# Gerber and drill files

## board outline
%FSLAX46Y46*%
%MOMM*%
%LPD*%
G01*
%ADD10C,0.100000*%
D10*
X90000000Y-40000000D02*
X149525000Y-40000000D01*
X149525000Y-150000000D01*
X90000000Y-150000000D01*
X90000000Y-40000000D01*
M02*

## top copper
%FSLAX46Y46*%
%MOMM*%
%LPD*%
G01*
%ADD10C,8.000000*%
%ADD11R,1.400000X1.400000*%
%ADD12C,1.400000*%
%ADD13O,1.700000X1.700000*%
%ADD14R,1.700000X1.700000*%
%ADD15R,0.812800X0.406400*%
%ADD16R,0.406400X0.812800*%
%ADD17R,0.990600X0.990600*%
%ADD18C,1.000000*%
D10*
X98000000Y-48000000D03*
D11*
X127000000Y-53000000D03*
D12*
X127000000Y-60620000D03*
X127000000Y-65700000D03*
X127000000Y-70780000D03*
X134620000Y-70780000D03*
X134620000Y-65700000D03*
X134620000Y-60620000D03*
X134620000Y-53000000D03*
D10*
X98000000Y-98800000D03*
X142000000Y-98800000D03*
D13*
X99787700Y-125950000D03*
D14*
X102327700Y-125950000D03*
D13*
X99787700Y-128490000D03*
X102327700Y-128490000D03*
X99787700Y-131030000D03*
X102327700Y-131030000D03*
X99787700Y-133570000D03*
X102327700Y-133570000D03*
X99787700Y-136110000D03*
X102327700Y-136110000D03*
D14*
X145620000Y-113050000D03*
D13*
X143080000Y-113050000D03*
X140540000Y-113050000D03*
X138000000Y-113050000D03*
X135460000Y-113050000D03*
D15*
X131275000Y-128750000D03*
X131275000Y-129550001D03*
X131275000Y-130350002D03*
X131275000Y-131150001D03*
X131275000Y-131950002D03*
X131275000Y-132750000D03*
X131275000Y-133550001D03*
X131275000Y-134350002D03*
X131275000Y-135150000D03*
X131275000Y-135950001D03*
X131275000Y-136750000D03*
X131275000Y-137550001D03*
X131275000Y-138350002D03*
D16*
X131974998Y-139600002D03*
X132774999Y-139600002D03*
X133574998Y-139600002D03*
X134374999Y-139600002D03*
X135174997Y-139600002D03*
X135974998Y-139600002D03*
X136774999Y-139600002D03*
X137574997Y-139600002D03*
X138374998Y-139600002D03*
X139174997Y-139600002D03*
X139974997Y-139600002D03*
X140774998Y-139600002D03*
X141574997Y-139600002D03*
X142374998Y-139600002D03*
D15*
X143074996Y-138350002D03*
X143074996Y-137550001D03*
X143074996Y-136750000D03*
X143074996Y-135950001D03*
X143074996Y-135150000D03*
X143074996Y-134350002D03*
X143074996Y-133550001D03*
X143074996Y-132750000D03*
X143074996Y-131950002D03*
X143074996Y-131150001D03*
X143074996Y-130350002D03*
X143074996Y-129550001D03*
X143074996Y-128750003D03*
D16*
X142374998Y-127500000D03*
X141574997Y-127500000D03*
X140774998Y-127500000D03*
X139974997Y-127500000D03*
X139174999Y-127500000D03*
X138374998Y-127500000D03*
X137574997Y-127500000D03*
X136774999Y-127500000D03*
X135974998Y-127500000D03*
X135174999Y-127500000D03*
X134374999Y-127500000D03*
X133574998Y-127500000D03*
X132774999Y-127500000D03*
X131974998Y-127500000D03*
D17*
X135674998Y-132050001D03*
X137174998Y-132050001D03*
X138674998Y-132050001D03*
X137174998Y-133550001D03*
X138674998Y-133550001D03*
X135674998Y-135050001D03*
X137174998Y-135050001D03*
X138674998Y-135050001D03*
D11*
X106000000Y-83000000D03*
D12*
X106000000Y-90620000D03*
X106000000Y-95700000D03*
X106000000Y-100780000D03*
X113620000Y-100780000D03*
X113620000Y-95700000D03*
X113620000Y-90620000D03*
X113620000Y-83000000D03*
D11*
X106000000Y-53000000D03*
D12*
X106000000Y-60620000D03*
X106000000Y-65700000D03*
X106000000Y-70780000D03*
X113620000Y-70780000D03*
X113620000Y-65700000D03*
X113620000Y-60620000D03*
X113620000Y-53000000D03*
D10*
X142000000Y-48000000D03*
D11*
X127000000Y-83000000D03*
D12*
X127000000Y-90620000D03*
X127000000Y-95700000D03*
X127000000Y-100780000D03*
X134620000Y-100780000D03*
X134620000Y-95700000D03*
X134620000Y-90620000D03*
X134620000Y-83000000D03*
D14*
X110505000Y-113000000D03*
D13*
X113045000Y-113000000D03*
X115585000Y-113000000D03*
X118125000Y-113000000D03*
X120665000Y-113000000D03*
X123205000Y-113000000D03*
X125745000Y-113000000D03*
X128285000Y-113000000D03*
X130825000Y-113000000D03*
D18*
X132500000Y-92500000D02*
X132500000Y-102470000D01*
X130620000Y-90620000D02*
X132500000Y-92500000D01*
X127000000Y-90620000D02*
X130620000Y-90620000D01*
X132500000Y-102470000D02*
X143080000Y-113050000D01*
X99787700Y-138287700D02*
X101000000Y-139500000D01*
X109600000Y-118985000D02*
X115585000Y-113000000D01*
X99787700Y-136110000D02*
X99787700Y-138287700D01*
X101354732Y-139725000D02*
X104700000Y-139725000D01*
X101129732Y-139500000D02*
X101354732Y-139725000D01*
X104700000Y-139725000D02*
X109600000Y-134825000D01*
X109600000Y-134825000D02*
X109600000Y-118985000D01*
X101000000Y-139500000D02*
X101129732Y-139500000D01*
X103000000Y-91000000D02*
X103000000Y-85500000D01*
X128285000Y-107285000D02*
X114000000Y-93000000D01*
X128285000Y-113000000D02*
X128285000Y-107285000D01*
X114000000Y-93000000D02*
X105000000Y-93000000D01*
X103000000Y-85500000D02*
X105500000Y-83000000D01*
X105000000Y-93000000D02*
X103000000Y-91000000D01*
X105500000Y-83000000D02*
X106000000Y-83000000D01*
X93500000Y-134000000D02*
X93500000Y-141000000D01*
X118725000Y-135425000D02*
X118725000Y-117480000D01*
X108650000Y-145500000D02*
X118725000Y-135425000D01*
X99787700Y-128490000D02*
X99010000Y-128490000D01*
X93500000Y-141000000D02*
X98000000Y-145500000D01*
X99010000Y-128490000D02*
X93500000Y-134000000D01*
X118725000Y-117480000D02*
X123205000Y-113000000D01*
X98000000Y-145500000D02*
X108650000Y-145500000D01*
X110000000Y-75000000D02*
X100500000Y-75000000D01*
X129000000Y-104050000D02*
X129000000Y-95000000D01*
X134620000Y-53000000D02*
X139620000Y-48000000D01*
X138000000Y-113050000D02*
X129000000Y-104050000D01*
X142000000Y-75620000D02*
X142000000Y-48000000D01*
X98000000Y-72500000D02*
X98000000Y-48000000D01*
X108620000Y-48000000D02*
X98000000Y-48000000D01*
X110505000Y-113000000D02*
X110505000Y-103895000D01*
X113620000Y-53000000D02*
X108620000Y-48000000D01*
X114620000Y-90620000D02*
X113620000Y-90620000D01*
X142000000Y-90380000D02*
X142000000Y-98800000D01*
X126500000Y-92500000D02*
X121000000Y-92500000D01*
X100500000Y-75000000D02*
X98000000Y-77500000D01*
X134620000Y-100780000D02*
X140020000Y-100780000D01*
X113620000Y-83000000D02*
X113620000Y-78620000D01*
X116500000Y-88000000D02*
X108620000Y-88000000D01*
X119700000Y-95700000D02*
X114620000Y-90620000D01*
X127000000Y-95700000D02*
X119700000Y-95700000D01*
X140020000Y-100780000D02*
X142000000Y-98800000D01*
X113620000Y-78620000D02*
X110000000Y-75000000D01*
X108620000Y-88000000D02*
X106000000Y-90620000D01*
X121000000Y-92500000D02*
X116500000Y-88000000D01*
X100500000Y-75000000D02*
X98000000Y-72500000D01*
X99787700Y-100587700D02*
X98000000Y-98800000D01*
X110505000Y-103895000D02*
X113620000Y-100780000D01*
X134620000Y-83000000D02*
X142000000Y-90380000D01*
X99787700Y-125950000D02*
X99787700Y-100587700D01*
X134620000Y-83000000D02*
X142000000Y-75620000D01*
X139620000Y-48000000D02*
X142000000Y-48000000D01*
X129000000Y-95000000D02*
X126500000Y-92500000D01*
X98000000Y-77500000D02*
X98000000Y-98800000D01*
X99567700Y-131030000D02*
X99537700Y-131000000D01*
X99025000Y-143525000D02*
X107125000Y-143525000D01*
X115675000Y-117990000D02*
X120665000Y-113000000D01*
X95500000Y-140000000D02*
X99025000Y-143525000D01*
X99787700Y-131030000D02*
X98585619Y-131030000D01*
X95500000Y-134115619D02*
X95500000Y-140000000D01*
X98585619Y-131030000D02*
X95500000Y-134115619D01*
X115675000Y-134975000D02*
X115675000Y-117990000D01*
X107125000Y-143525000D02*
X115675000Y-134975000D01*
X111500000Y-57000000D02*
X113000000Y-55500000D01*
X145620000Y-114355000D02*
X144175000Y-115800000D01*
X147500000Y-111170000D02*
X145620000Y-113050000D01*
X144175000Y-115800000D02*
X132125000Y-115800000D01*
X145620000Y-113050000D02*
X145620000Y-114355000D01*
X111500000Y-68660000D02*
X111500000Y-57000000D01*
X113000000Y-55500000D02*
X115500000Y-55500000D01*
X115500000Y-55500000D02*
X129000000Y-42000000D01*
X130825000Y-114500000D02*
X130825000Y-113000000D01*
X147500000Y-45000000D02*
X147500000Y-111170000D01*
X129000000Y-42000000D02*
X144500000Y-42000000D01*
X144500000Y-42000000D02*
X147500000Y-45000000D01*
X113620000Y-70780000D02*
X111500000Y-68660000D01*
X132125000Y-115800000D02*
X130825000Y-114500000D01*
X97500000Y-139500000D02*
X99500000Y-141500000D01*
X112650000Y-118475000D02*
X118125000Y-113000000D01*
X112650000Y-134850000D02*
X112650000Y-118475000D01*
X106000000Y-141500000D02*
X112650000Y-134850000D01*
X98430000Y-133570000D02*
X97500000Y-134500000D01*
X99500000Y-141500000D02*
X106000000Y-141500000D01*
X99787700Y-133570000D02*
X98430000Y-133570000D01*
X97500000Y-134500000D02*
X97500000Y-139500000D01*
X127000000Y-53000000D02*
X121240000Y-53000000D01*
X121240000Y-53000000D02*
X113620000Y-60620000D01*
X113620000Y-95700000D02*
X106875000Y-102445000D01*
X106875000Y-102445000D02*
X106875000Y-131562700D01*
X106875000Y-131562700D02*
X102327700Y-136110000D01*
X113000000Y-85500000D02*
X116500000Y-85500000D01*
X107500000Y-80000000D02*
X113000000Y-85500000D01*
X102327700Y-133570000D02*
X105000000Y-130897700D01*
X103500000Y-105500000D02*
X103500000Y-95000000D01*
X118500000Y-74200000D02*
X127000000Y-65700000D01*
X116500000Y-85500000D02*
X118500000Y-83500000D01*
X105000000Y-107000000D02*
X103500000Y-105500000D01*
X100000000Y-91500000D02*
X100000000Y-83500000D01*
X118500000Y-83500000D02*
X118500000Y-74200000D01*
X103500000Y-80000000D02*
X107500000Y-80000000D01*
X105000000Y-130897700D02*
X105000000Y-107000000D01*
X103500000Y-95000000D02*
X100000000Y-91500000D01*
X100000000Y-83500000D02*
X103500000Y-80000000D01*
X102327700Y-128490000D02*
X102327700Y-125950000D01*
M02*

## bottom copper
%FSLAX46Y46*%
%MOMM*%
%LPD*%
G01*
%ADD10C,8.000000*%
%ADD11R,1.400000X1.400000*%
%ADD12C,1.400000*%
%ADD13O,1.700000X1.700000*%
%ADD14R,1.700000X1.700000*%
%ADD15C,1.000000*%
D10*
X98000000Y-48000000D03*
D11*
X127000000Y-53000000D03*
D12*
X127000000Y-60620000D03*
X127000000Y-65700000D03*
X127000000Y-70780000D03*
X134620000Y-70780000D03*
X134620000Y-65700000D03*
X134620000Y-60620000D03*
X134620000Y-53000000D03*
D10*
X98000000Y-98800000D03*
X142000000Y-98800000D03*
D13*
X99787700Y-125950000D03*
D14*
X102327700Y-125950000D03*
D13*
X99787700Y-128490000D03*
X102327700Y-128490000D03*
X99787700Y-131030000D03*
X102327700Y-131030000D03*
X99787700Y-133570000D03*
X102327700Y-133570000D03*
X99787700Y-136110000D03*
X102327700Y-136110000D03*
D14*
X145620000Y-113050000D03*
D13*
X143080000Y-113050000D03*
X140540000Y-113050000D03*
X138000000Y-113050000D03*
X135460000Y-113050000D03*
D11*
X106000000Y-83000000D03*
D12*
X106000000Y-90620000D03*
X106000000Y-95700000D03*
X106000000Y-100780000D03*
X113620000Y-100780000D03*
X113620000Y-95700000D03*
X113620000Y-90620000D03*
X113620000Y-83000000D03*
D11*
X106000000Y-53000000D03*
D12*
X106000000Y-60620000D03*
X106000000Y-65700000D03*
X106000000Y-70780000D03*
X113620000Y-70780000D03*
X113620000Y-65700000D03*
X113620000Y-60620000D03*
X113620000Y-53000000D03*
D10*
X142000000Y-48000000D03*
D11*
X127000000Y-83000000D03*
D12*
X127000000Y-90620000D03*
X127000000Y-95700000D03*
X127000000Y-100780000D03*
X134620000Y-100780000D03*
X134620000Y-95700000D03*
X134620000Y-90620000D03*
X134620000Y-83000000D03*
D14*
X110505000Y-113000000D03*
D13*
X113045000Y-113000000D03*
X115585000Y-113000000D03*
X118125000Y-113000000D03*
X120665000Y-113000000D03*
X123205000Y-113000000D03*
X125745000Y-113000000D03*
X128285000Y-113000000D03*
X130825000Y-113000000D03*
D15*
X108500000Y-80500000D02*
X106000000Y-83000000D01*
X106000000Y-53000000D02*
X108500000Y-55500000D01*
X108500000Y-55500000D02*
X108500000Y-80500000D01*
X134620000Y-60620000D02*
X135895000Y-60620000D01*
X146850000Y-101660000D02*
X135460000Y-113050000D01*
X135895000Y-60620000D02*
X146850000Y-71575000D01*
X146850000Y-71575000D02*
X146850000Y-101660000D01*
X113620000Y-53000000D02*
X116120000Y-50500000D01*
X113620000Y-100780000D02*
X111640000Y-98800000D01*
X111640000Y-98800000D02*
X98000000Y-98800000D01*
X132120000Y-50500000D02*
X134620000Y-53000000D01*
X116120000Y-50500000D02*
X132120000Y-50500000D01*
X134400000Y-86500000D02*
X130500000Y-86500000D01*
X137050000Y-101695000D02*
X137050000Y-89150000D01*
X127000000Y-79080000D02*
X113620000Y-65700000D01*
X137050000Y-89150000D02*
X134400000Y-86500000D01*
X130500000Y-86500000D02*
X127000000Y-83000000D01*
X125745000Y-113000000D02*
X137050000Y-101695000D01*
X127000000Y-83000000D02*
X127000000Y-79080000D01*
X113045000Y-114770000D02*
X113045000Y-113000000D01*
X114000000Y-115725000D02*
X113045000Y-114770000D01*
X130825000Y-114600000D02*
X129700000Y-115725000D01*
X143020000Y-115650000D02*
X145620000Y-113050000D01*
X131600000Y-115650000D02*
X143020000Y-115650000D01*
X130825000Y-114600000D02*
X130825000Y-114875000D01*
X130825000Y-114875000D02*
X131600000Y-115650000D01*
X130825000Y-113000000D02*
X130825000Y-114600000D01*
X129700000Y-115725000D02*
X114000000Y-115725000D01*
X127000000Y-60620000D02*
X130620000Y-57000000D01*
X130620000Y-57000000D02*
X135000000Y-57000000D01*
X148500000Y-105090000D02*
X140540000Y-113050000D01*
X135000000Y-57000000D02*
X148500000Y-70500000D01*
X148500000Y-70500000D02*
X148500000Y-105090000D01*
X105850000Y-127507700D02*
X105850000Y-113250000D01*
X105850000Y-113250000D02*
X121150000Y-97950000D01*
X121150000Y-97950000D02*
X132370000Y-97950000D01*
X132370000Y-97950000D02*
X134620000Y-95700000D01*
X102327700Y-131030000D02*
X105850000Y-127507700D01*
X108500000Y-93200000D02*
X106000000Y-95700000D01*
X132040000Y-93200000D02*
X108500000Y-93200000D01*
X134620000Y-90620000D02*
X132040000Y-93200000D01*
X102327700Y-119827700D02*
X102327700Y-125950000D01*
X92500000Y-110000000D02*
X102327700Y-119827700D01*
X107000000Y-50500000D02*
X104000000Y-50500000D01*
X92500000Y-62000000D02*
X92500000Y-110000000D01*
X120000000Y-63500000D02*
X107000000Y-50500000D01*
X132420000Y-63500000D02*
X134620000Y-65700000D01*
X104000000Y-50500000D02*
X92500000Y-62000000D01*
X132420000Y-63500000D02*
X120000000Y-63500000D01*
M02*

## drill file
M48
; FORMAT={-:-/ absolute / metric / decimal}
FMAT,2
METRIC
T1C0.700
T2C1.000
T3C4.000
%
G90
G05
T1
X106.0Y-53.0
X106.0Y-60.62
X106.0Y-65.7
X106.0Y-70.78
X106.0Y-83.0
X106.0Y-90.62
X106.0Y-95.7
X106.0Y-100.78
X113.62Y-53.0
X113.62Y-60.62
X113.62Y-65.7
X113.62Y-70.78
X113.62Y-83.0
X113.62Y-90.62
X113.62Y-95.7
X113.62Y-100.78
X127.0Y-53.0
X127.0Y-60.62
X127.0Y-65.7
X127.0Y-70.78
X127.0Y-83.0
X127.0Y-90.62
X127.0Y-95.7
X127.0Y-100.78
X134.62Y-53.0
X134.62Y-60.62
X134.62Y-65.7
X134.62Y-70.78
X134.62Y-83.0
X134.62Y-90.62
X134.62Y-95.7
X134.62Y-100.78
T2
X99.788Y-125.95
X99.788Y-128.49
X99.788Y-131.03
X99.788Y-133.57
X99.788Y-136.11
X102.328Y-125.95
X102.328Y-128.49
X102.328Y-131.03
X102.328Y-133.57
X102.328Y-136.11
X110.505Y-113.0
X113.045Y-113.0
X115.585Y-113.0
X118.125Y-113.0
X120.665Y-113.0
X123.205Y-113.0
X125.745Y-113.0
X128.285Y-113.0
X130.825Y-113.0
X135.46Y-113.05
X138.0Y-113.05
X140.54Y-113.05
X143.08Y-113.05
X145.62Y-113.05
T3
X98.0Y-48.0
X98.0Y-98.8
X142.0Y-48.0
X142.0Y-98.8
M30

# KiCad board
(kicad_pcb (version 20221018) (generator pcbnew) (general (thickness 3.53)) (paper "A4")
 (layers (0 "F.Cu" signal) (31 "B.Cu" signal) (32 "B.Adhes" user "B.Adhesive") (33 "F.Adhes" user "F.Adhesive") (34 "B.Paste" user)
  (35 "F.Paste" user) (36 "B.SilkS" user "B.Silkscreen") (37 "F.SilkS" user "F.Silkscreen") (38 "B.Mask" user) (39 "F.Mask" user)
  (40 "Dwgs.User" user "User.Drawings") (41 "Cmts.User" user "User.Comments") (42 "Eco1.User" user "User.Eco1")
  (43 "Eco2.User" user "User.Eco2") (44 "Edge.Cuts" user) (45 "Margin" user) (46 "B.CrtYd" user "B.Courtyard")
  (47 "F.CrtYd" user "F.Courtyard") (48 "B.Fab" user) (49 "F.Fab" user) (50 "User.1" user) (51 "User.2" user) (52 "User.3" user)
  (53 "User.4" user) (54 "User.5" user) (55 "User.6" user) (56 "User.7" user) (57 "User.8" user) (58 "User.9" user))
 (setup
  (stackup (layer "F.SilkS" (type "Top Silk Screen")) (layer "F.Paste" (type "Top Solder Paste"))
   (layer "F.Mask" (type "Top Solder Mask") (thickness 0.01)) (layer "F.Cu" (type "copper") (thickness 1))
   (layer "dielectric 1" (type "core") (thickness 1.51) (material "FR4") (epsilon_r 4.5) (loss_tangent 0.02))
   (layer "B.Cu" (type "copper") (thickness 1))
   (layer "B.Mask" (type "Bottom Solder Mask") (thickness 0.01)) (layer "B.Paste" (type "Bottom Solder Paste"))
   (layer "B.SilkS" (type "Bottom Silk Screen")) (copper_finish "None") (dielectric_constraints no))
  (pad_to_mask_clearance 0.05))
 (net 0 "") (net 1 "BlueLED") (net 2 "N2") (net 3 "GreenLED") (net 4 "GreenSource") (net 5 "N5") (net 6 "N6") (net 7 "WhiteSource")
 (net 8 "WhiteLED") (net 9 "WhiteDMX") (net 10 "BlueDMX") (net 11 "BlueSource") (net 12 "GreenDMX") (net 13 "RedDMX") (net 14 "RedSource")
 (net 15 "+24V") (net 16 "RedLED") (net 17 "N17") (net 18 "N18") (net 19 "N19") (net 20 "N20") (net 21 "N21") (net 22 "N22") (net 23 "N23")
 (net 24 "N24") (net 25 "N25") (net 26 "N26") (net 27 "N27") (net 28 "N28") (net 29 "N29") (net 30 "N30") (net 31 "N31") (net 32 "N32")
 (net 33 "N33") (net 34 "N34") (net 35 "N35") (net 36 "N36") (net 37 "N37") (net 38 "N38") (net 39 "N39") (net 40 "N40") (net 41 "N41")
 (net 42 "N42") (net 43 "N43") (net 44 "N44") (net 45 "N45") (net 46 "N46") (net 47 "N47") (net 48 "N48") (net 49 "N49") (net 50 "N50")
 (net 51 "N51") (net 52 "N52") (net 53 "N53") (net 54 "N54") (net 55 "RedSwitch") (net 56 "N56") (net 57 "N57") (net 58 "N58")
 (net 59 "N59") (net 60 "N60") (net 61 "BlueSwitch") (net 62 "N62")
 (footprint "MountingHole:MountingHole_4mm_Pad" (layer "F.Cu") (at 98 48)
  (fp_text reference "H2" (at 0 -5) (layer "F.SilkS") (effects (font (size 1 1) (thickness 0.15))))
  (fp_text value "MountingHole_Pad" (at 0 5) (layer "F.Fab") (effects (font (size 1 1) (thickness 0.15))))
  (pad "1" thru_hole circle (at 0 0) (size 8 8) (drill 4) (layers "*.Cu" "*.Mask") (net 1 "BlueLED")))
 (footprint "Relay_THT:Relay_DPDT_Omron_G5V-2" (layer "F.Cu") (at 127 53)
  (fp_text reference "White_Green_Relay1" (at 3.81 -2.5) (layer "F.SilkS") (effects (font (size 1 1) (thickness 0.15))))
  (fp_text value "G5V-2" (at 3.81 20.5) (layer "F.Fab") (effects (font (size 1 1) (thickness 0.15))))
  (pad "1" thru_hole rect (at 0 0) (size 1.4 1.4) (drill 0.7) (layers "*.Cu" "*.Mask") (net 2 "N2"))
  (pad "4" thru_hole circle (at 0 7.62) (size 1.4 1.4) (drill 0.7) (layers "*.Cu" "*.Mask") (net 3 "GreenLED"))
  (pad "6" thru_hole circle (at 0 12.7) (size 1.4 1.4) (drill 0.7) (layers "*.Cu" "*.Mask") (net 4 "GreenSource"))
  (pad "8" thru_hole circle (at 0 17.78) (size 1.4 1.4) (drill 0.7) (layers "*.Cu" "*.Mask") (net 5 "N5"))
  (pad "9" thru_hole circle (at 7.62 17.78) (size 1.4 1.4) (drill 0.7) (layers "*.Cu" "*.Mask") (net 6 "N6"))
  (pad "11" thru_hole circle (at 7.62 12.7) (size 1.4 1.4) (drill 0.7) (layers "*.Cu" "*.Mask") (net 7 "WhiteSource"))
  (pad "13" thru_hole circle (at 7.62 7.62) (size 1.4 1.4) (drill 0.7) (layers "*.Cu" "*.Mask") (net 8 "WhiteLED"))
  (pad "16" thru_hole circle (at 7.62 0) (size 1.4 1.4) (drill 0.7) (layers "*.Cu" "*.Mask") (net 1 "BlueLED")))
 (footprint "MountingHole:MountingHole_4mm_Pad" (layer "F.Cu") (at 98 98.8)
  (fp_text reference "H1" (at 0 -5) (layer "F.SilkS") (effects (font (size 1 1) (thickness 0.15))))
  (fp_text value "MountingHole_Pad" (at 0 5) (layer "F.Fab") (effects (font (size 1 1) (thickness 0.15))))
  (pad "1" thru_hole circle (at 0 0) (size 8 8) (drill 4) (layers "*.Cu" "*.Mask") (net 1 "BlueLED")))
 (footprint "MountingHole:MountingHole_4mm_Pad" (layer "F.Cu") (at 142 98.8)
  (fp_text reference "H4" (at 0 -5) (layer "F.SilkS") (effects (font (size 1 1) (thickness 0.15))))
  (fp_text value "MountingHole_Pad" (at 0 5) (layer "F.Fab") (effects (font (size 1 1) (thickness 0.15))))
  (pad "1" thru_hole circle (at 0 0) (size 8 8) (drill 4) (layers "*.Cu" "*.Mask") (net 1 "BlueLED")))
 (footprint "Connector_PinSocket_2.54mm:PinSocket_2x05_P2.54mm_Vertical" (layer "F.Cu") (at 102.3277 125.95)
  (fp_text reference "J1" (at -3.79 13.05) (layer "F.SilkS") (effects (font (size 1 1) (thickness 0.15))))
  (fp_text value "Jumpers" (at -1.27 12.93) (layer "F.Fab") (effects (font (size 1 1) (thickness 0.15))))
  (pad "1a" thru_hole oval (at -2.54 0) (size 1.7 1.7) (drill 1) (layers "*.Cu" "*.Mask") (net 1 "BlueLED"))
  (pad "1b" thru_hole rect (at 0 0) (size 1.7 1.7) (drill 1) (layers "*.Cu" "*.Mask") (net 7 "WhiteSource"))
  (pad "2a" thru_hole oval (at -2.54 2.54) (size 1.7 1.7) (drill 1) (layers "*.Cu" "*.Mask") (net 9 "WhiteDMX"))
  (pad "2b" thru_hole oval (at 0 2.54) (size 1.7 1.7) (drill 1) (layers "*.Cu" "*.Mask") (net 7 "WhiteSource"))
  (pad "3a" thru_hole oval (at -2.54 5.08) (size 1.7 1.7) (drill 1) (layers "*.Cu" "*.Mask") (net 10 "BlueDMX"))
  (pad "3b" thru_hole oval (at 0 5.08) (size 1.7 1.7) (drill 1) (layers "*.Cu" "*.Mask") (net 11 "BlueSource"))
  (pad "4a" thru_hole oval (at -2.54 7.62) (size 1.7 1.7) (drill 1) (layers "*.Cu" "*.Mask") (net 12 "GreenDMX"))
  (pad "4b" thru_hole oval (at 0 7.62) (size 1.7 1.7) (drill 1) (layers "*.Cu" "*.Mask") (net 4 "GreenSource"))
  (pad "5a" thru_hole oval (at -2.54 10.16) (size 1.7 1.7) (drill 1) (layers "*.Cu" "*.Mask") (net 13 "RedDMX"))
  (pad "5b" thru_hole oval (at 0 10.16) (size 1.7 1.7) (drill 1) (layers "*.Cu" "*.Mask") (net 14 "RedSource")))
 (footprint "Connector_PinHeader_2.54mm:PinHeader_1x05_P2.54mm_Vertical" (layer "F.Cu") (at 145.62 113.05 -90)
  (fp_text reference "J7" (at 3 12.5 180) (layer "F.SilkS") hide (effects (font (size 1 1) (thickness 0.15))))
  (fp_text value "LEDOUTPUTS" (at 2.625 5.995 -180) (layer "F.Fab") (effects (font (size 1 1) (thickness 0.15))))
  (pad "1" thru_hole rect (at 0 0 270) (size 1.7 1.7) (drill 1) (layers "*.Cu" "*.Mask") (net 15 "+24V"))
  (pad "2" thru_hole oval (at 0 2.54 270) (size 1.7 1.7) (drill 1) (layers "*.Cu" "*.Mask") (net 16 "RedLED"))
  (pad "3" thru_hole oval (at 0 5.08 270) (size 1.7 1.7) (drill 1) (layers "*.Cu" "*.Mask") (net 3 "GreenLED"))
  (pad "4" thru_hole oval (at 0 7.62 270) (size 1.7 1.7) (drill 1) (layers "*.Cu" "*.Mask") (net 1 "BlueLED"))
  (pad "5" thru_hole oval (at 0 10.16 270) (size 1.7 1.7) (drill 1) (layers "*.Cu" "*.Mask") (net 8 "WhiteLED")))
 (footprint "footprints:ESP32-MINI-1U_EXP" (layer "F.Cu") (at 137.174998 133.550001)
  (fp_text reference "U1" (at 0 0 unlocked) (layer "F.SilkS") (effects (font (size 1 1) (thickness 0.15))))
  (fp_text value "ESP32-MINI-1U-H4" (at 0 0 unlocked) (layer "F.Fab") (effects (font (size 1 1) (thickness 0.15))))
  (pad "1" smd rect (at -5.899998 -4.800001) (size 0.8128 0.4064) (layers "F.Cu" "F.Paste" "F.Mask") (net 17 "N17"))
  (pad "2" smd rect (at -5.899998 -4) (size 0.8128 0.4064) (layers "F.Cu" "F.Paste" "F.Mask") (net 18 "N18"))
  (pad "3" smd rect (at -5.899998 -3.199999) (size 0.8128 0.4064) (layers "F.Cu" "F.Paste" "F.Mask") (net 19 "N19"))
  (pad "4" smd rect (at -5.899998 -2.4) (size 0.8128 0.4064) (layers "F.Cu" "F.Paste" "F.Mask") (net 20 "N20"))
  (pad "5" smd rect (at -5.899998 -1.599999) (size 0.8128 0.4064) (layers "F.Cu" "F.Paste" "F.Mask") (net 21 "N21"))
  (pad "6" smd rect (at -5.899998 -0.800001) (size 0.8128 0.4064) (layers "F.Cu" "F.Paste" "F.Mask") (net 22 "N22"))
  (pad "7" smd rect (at -5.899998 0) (size 0.8128 0.4064) (layers "F.Cu" "F.Paste" "F.Mask") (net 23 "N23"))
  (pad "8" smd rect (at -5.899998 0.800001) (size 0.8128 0.4064) (layers "F.Cu" "F.Paste" "F.Mask") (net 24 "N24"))
  (pad "9" smd rect (at -5.899998 1.599999) (size 0.8128 0.4064) (layers "F.Cu" "F.Paste" "F.Mask") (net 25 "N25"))
  (pad "10" smd rect (at -5.899998 2.4) (size 0.8128 0.4064) (layers "F.Cu" "F.Paste" "F.Mask") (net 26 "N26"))
  (pad "11" smd rect (at -5.899998 3.199999) (size 0.8128 0.4064) (layers "F.Cu" "F.Paste" "F.Mask") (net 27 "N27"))
  (pad "12" smd rect (at -5.899998 4) (size 0.8128 0.4064) (layers "F.Cu" "F.Paste" "F.Mask") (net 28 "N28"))
  (pad "13" smd rect (at -5.899998 4.800001) (size 0.8128 0.4064) (layers "F.Cu" "F.Paste" "F.Mask") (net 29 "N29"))
  (pad "14" smd rect (at -5.2 6.050001 90) (size 0.8128 0.4064) (layers "F.Cu" "F.Paste" "F.Mask") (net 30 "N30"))
  (pad "15" smd rect (at -4.399999 6.050001 90) (size 0.8128 0.4064) (layers "F.Cu" "F.Paste" "F.Mask") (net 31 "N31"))
  (pad "16" smd rect (at -3.6 6.050001 90) (size 0.8128 0.4064) (layers "F.Cu" "F.Paste" "F.Mask") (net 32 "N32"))
  (pad "17" smd rect (at -2.799999 6.050001 90) (size 0.8128 0.4064) (layers "F.Cu" "F.Paste" "F.Mask") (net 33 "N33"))
  (pad "18" smd rect (at -2.000001 6.050001 90) (size 0.8128 0.4064) (layers "F.Cu" "F.Paste" "F.Mask") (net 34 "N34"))
  (pad "19" smd rect (at -1.2 6.050001 90) (size 0.8128 0.4064) (layers "F.Cu" "F.Paste" "F.Mask") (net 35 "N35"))
  (pad "20" smd rect (at -0.399999 6.050001 90) (size 0.8128 0.4064) (layers "F.Cu" "F.Paste" "F.Mask") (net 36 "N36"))
  (pad "21" smd rect (at 0.399999 6.050001 90) (size 0.8128 0.4064) (layers "F.Cu" "F.Paste" "F.Mask") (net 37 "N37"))
  (pad "22" smd rect (at 1.2 6.050001 90) (size 0.8128 0.4064) (layers "F.Cu" "F.Paste" "F.Mask") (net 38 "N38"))
  (pad "23" smd rect (at 1.999999 6.050001 90) (size 0.8128 0.4064) (layers "F.Cu" "F.Paste" "F.Mask") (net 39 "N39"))
  (pad "24" smd rect (at 2.799999 6.050001 90) (size 0.8128 0.4064) (layers "F.Cu" "F.Paste" "F.Mask") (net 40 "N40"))
  (pad "25" smd rect (at 3.6 6.050001 90) (size 0.8128 0.4064) (layers "F.Cu" "F.Paste" "F.Mask") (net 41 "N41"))
  (pad "26" smd rect (at 4.399999 6.050001 90) (size 0.8128 0.4064) (layers "F.Cu" "F.Paste" "F.Mask") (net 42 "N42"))
  (pad "27" smd rect (at 5.2 6.050001 90) (size 0.8128 0.4064) (layers "F.Cu" "F.Paste" "F.Mask") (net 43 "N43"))
  (pad "28" smd rect (at 5.899998 4.800001) (size 0.8128 0.4064) (layers "F.Cu" "F.Paste" "F.Mask") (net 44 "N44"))
  (pad "29" smd rect (at 5.899998 4) (size 0.8128 0.4064) (layers "F.Cu" "F.Paste" "F.Mask") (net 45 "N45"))
  (pad "30" smd rect (at 5.899998 3.199999) (size 0.8128 0.4064) (layers "F.Cu" "F.Paste" "F.Mask") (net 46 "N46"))
  (pad "31" smd rect (at 5.899998 2.4) (size 0.8128 0.4064) (layers "F.Cu" "F.Paste" "F.Mask") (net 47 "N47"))
  (pad "32" smd rect (at 5.899998 1.599999) (size 0.8128 0.4064) (layers "F.Cu" "F.Paste" "F.Mask") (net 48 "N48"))
  (pad "33" smd rect (at 5.899998 0.800001) (size 0.8128 0.4064) (layers "F.Cu" "F.Paste" "F.Mask") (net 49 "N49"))
  (pad "34" smd rect (at 5.899998 0) (size 0.8128 0.4064) (layers "F.Cu" "F.Paste" "F.Mask") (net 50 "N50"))
  (pad "35" smd rect (at 5.899998 -0.800001) (size 0.8128 0.4064) (layers "F.Cu" "F.Paste" "F.Mask") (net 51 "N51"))
  (pad "36" smd rect (at 5.899998 -1.599999) (size 0.8128 0.4064) (layers "F.Cu" "F.Paste" "F.Mask") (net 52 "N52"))
  (pad "37" smd rect (at 5.899998 -2.4) (size 0.8128 0.4064) (layers "F.Cu" "F.Paste" "F.Mask") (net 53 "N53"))
  (pad "38" smd rect (at 5.899998 -3.199999) (size 0.8128 0.4064) (layers "F.Cu" "F.Paste" "F.Mask") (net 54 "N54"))
  (pad "39" smd rect (at 5.899998 -4) (size 0.8128 0.4064) (layers "F.Cu" "F.Paste" "F.Mask") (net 54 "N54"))
  (pad "40" smd rect (at 5.899998 -4.799998) (size 0.8128 0.4064) (layers "F.Cu" "F.Paste" "F.Mask") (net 54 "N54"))
  (pad "41" smd rect (at 5.2 -6.050001 90) (size 0.8128 0.4064) (layers "F.Cu" "F.Paste" "F.Mask") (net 54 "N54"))
  (pad "42" smd rect (at 4.399999 -6.050001 90) (size 0.8128 0.4064) (layers "F.Cu" "F.Paste" "F.Mask") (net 54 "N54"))
  (pad "43" smd rect (at 3.6 -6.050001 90) (size 0.8128 0.4064) (layers "F.Cu" "F.Paste" "F.Mask") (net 54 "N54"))
  (pad "44" smd rect (at 2.799999 -6.050001 90) (size 0.8128 0.4064) (layers "F.Cu" "F.Paste" "F.Mask") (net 54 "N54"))
  (pad "45" smd rect (at 2.000001 -6.050001 90) (size 0.8128 0.4064) (layers "F.Cu" "F.Paste" "F.Mask") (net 54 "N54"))
  (pad "46" smd rect (at 1.2 -6.050001 90) (size 0.8128 0.4064) (layers "F.Cu" "F.Paste" "F.Mask") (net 54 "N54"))
  (pad "47" smd rect (at 0.399999 -6.050001 90) (size 0.8128 0.4064) (layers "F.Cu" "F.Paste" "F.Mask") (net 54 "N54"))
  (pad "48" smd rect (at -0.399999 -6.050001 90) (size 0.8128 0.4064) (layers "F.Cu" "F.Paste" "F.Mask") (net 54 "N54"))
  (pad "49" smd rect (at -1.2 -6.050001 90) (size 0.8128 0.4064) (layers "F.Cu" "F.Paste" "F.Mask") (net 54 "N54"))
  (pad "50" smd rect (at -1.999999 -6.050001 90) (size 0.8128 0.4064) (layers "F.Cu" "F.Paste" "F.Mask") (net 54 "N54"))
  (pad "51" smd rect (at -2.799999 -6.050001 90) (size 0.8128 0.4064) (layers "F.Cu" "F.Paste" "F.Mask") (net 54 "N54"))
  (pad "52" smd rect (at -3.6 -6.050001 90) (size 0.8128 0.4064) (layers "F.Cu" "F.Paste" "F.Mask") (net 54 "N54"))
  (pad "53" smd rect (at -4.399999 -6.050001 90) (size 0.8128 0.4064) (layers "F.Cu" "F.Paste" "F.Mask") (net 54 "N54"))
  (pad "54" smd rect (at -5.2 -6.050001 90) (size 0.8128 0.4064) (layers "F.Cu" "F.Paste" "F.Mask") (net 54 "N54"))
  (pad "55" smd rect (at -1.5 -1.5) (size 0.9906 0.9906) (layers "F.Cu" "F.Paste" "F.Mask") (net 54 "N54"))
  (pad "56" smd rect (at 0 -1.5) (size 0.9906 0.9906) (layers "F.Cu" "F.Paste" "F.Mask") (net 54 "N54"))
  (pad "57" smd rect (at 1.5 -1.5) (size 0.9906 0.9906) (layers "F.Cu" "F.Paste" "F.Mask") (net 54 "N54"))
  (pad "58" smd rect (at 0 0) (size 0.9906 0.9906) (layers "F.Cu" "F.Paste" "F.Mask") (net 54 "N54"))
  (pad "59" smd rect (at 1.5 0) (size 0.9906 0.9906) (layers "F.Cu" "F.Paste" "F.Mask") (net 54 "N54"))
  (pad "60" smd rect (at -1.5 1.5) (size 0.9906 0.9906) (layers "F.Cu" "F.Paste" "F.Mask") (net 54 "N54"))
  (pad "61" smd rect (at 0 1.5) (size 0.9906 0.9906) (layers "F.Cu" "F.Paste" "F.Mask") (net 54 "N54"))
  (pad "62" smd rect (at 1.5 1.5) (size 0.9906 0.9906) (layers "F.Cu" "F.Paste" "F.Mask") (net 54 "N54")))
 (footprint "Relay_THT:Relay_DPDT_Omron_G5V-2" (layer "F.Cu") (at 106 83)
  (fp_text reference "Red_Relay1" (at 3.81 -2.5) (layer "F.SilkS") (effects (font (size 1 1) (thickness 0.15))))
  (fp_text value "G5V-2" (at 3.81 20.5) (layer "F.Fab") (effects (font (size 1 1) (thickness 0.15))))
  (pad "1" thru_hole rect (at 0 0) (size 1.4 1.4) (drill 0.7) (layers "*.Cu" "*.Mask") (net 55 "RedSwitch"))
  (pad "4" thru_hole circle (at 0 7.62) (size 1.4 1.4) (drill 0.7) (layers "*.Cu" "*.Mask") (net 1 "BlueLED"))
  (pad "6" thru_hole circle (at 0 12.7) (size 1.4 1.4) (drill 0.7) (layers "*.Cu" "*.Mask") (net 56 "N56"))
  (pad "8" thru_hole circle (at 0 17.78) (size 1.4 1.4) (drill 0.7) (layers "*.Cu" "*.Mask") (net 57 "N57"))
  (pad "9" thru_hole circle (at 7.62 17.78) (size 1.4 1.4) (drill 0.7) (layers "*.Cu" "*.Mask") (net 1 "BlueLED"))
  (pad "11" thru_hole circle (at 7.62 12.7) (size 1.4 1.4) (drill 0.7) (layers "*.Cu" "*.Mask") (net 14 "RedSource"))
  (pad "13" thru_hole circle (at 7.62 7.62) (size 1.4 1.4) (drill 0.7) (layers "*.Cu" "*.Mask") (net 1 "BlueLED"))
  (pad "16" thru_hole circle (at 7.62 0) (size 1.4 1.4) (drill 0.7) (layers "*.Cu" "*.Mask") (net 1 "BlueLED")))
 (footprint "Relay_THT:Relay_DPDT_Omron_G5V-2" (layer "F.Cu") (at 106 53)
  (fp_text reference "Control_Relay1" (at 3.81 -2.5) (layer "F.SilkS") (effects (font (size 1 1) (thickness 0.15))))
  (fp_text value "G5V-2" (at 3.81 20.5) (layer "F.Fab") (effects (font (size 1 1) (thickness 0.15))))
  (pad "1" thru_hole rect (at 0 0) (size 1.4 1.4) (drill 0.7) (layers "*.Cu" "*.Mask") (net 55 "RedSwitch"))
  (pad "4" thru_hole circle (at 0 7.62) (size 1.4 1.4) (drill 0.7) (layers "*.Cu" "*.Mask") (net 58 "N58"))
  (pad "6" thru_hole circle (at 0 12.7) (size 1.4 1.4) (drill 0.7) (layers "*.Cu" "*.Mask") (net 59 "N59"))
  (pad "8" thru_hole circle (at 0 17.78) (size 1.4 1.4) (drill 0.7) (layers "*.Cu" "*.Mask") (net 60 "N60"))
  (pad "9" thru_hole circle (at 7.62 17.78) (size 1.4 1.4) (drill 0.7) (layers "*.Cu" "*.Mask") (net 15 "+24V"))
  (pad "11" thru_hole circle (at 7.62 12.7) (size 1.4 1.4) (drill 0.7) (layers "*.Cu" "*.Mask") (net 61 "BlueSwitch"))
  (pad "13" thru_hole circle (at 7.62 7.62) (size 1.4 1.4) (drill 0.7) (layers "*.Cu" "*.Mask") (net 2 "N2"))
  (pad "16" thru_hole circle (at 7.62 0) (size 1.4 1.4) (drill 0.7) (layers "*.Cu" "*.Mask") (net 1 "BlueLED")))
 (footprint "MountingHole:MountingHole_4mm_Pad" (layer "F.Cu") (at 142 48)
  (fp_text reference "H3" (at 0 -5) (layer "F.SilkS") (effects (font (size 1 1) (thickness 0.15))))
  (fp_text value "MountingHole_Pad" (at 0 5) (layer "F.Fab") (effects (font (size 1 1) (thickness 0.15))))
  (pad "1" thru_hole circle (at 0 0) (size 8 8) (drill 4) (layers "*.Cu" "*.Mask") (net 1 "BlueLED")))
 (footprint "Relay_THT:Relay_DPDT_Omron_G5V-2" (layer "F.Cu") (at 127 83)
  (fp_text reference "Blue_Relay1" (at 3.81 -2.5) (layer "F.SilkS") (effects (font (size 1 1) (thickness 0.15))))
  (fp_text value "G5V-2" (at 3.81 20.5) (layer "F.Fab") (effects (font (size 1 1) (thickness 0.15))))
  (pad "1" thru_hole rect (at 0 0) (size 1.4 1.4) (drill 0.7) (layers "*.Cu" "*.Mask") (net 61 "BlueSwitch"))
  (pad "4" thru_hole circle (at 0 7.62) (size 1.4 1.4) (drill 0.7) (layers "*.Cu" "*.Mask") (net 16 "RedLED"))
  (pad "6" thru_hole circle (at 0 12.7) (size 1.4 1.4) (drill 0.7) (layers "*.Cu" "*.Mask") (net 1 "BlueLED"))
  (pad "8" thru_hole circle (at 0 17.78) (size 1.4 1.4) (drill 0.7) (layers "*.Cu" "*.Mask") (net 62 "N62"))
  (pad "9" thru_hole circle (at 7.62 17.78) (size 1.4 1.4) (drill 0.7) (layers "*.Cu" "*.Mask") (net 1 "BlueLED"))
  (pad "11" thru_hole circle (at 7.62 12.7) (size 1.4 1.4) (drill 0.7) (layers "*.Cu" "*.Mask") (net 11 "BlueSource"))
  (pad "13" thru_hole circle (at 7.62 7.62) (size 1.4 1.4) (drill 0.7) (layers "*.Cu" "*.Mask") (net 56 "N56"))
  (pad "16" thru_hole circle (at 7.62 0) (size 1.4 1.4) (drill 0.7) (layers "*.Cu" "*.Mask") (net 1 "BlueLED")))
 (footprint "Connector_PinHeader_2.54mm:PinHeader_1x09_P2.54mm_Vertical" (layer "F.Cu") (at 110.505 113 90)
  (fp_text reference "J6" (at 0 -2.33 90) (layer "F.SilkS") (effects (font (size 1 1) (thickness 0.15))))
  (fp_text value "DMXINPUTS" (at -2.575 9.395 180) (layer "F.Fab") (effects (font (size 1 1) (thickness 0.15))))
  (pad "1" thru_hole rect (at 0 0 90) (size 1.7 1.7) (drill 1) (layers "*.Cu" "*.Mask") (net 1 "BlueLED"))
  (pad "2" thru_hole oval (at 0 2.54 90) (size 1.7 1.7) (drill 1) (layers "*.Cu" "*.Mask") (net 15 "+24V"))
  (pad "3" thru_hole oval (at 0 5.08 90) (size 1.7 1.7) (drill 1) (layers "*.Cu" "*.Mask") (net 13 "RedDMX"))
  (pad "4" thru_hole oval (at 0 7.62 90) (size 1.7 1.7) (drill 1) (layers "*.Cu" "*.Mask") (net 12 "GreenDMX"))
  (pad "5" thru_hole oval (at 0 10.16 90) (size 1.7 1.7) (drill 1) (layers "*.Cu" "*.Mask") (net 10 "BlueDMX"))
  (pad "6" thru_hole oval (at 0 12.7 90) (size 1.7 1.7) (drill 1) (layers "*.Cu" "*.Mask") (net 9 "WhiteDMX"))
  (pad "7" thru_hole oval (at 0 15.24 90) (size 1.7 1.7) (drill 1) (layers "*.Cu" "*.Mask") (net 61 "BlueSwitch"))
  (pad "8" thru_hole oval (at 0 17.78 90) (size 1.7 1.7) (drill 1) (layers "*.Cu" "*.Mask") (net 55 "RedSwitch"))
  (pad "9" thru_hole oval (at 0 20.32 90) (size 1.7 1.7) (drill 1) (layers "*.Cu" "*.Mask") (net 15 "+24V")))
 (gr_rect (start 90 40) (end 149.525 150) (stroke (width 0.1) (type solid)) (fill none) (layer "Edge.Cuts"))
 (segment (start 132.5 92.5) (end 132.5 102.47) (width 1) (layer "F.Cu") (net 16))
 (segment (start 130.62 90.62) (end 132.5 92.5) (width 1) (layer "F.Cu") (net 16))
 (segment (start 127 90.62) (end 130.62 90.62) (width 1) (layer "F.Cu") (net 16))
 (segment (start 132.5 102.47) (end 143.08 113.05) (width 1) (layer "F.Cu") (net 16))
 (segment (start 99.7877 138.2877) (end 101 139.5) (width 1) (layer "F.Cu") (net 13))
 (segment (start 109.6 118.985) (end 115.585 113) (width 1) (layer "F.Cu") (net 13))
 (segment (start 99.7877 136.11) (end 99.7877 138.2877) (width 1) (layer "F.Cu") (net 13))
 (segment (start 101.354732 139.725) (end 104.7 139.725) (width 1) (layer "F.Cu") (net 13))
 (segment (start 101.129732 139.5) (end 101.354732 139.725) (width 1) (layer "F.Cu") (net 13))
 (segment (start 104.7 139.725) (end 109.6 134.825) (width 1) (layer "F.Cu") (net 13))
 (segment (start 109.6 134.825) (end 109.6 118.985) (width 1) (layer "F.Cu") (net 13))
 (segment (start 101 139.5) (end 101.129732 139.5) (width 1) (layer "F.Cu") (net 13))
 (segment (start 103 91) (end 103 85.5) (width 1) (layer "F.Cu") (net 55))
 (segment (start 128.285 107.285) (end 114 93) (width 1) (layer "F.Cu") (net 55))
 (segment (start 128.285 113) (end 128.285 107.285) (width 1) (layer "F.Cu") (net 55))
 (segment (start 114 93) (end 105 93) (width 1) (layer "F.Cu") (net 55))
 (segment (start 103 85.5) (end 105.5 83) (width 1) (layer "F.Cu") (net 55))
 (segment (start 105 93) (end 103 91) (width 1) (layer "F.Cu") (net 55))
 (segment (start 105.5 83) (end 106 83) (width 1) (layer "F.Cu") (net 55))
 (segment (start 108.5 80.5) (end 106 83) (width 1) (layer "B.Cu") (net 55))
 (segment (start 106 53) (end 108.5 55.5) (width 1) (layer "B.Cu") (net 55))
 (segment (start 108.5 55.5) (end 108.5 80.5) (width 1) (layer "B.Cu") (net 55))
 (segment (start 134.62 60.62) (end 135.895 60.62) (width 1) (layer "B.Cu") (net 8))
 (segment (start 146.85 101.66) (end 135.46 113.05) (width 1) (layer "B.Cu") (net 8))
 (segment (start 135.895 60.62) (end 146.85 71.575) (width 1) (layer "B.Cu") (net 8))
 (segment (start 146.85 71.575) (end 146.85 101.66) (width 1) (layer "B.Cu") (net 8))
 (segment (start 93.5 134) (end 93.5 141) (width 1) (layer "F.Cu") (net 9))
 (segment (start 118.725 135.425) (end 118.725 117.48) (width 1) (layer "F.Cu") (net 9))
 (segment (start 108.65 145.5) (end 118.725 135.425) (width 1) (layer "F.Cu") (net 9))
 (segment (start 99.7877 128.49) (end 99.01 128.49) (width 1) (layer "F.Cu") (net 9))
 (segment (start 93.5 141) (end 98 145.5) (width 1) (layer "F.Cu") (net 9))
 (segment (start 99.01 128.49) (end 93.5 134) (width 1) (layer "F.Cu") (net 9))
 (segment (start 118.725 117.48) (end 123.205 113) (width 1) (layer "F.Cu") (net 9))
 (segment (start 98 145.5) (end 108.65 145.5) (width 1) (layer "F.Cu") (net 9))
 (segment (start 110 75) (end 100.5 75) (width 1) (layer "F.Cu") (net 1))
 (segment (start 129 104.05) (end 129 95) (width 1) (layer "F.Cu") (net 1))
 (segment (start 134.62 53) (end 139.62 48) (width 1) (layer "F.Cu") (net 1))
 (segment (start 138 113.05) (end 129 104.05) (width 1) (layer "F.Cu") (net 1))
 (segment (start 142 75.62) (end 142 48) (width 1) (layer "F.Cu") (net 1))
 (segment (start 98 72.5) (end 98 48) (width 1) (layer "F.Cu") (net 1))
 (segment (start 108.62 48) (end 98 48) (width 1) (layer "F.Cu") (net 1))
 (segment (start 110.505 113) (end 110.505 103.895) (width 1) (layer "F.Cu") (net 1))
 (segment (start 113.62 53) (end 108.62 48) (width 1) (layer "F.Cu") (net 1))
 (segment (start 114.62 90.62) (end 113.62 90.62) (width 1) (layer "F.Cu") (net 1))
 (segment (start 142 90.38) (end 142 98.8) (width 1) (layer "F.Cu") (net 1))
 (segment (start 126.5 92.5) (end 121 92.5) (width 1) (layer "F.Cu") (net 1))
 (segment (start 100.5 75) (end 98 77.5) (width 1) (layer "F.Cu") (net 1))
 (segment (start 134.62 100.78) (end 140.02 100.78) (width 1) (layer "F.Cu") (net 1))
 (segment (start 113.62 83) (end 113.62 78.62) (width 1) (layer "F.Cu") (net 1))
 (segment (start 116.5 88) (end 108.62 88) (width 1) (layer "F.Cu") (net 1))
 (segment (start 119.7 95.7) (end 114.62 90.62) (width 1) (layer "F.Cu") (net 1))
 (segment (start 127 95.7) (end 119.7 95.7) (width 1) (layer "F.Cu") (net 1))
 (segment (start 140.02 100.78) (end 142 98.8) (width 1) (layer "F.Cu") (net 1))
 (segment (start 113.62 78.62) (end 110 75) (width 1) (layer "F.Cu") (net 1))
 (segment (start 108.62 88) (end 106 90.62) (width 1) (layer "F.Cu") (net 1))
 (segment (start 121 92.5) (end 116.5 88) (width 1) (layer "F.Cu") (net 1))
 (segment (start 100.5 75) (end 98 72.5) (width 1) (layer "F.Cu") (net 1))
 (segment (start 99.7877 100.5877) (end 98 98.8) (width 1) (layer "F.Cu") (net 1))
 (segment (start 110.505 103.895) (end 113.62 100.78) (width 1) (layer "F.Cu") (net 1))
 (segment (start 134.62 83) (end 142 90.38) (width 1) (layer "F.Cu") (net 1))
 (segment (start 99.7877 125.95) (end 99.7877 100.5877) (width 1) (layer "F.Cu") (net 1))
 (segment (start 134.62 83) (end 142 75.62) (width 1) (layer "F.Cu") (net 1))
 (segment (start 139.62 48) (end 142 48) (width 1) (layer "F.Cu") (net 1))
 (segment (start 129 95) (end 126.5 92.5) (width 1) (layer "F.Cu") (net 1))
 (segment (start 98 77.5) (end 98 98.8) (width 1) (layer "F.Cu") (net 1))
 (segment (start 113.62 53) (end 116.12 50.5) (width 1) (layer "B.Cu") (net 1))
 (segment (start 113.62 100.78) (end 111.64 98.8) (width 1) (layer "B.Cu") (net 1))
 (segment (start 111.64 98.8) (end 98 98.8) (width 1) (layer "B.Cu") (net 1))
 (segment (start 132.12 50.5) (end 134.62 53) (width 1) (layer "B.Cu") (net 1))
 (segment (start 116.12 50.5) (end 132.12 50.5) (width 1) (layer "B.Cu") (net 1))
 (segment (start 99.5677 131.03) (end 99.5377 131) (width 1) (layer "F.Cu") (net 10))
 (segment (start 99.025 143.525) (end 107.125 143.525) (width 1) (layer "F.Cu") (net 10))
 (segment (start 115.675 117.99) (end 120.665 113) (width 1) (layer "F.Cu") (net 10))
 (segment (start 95.5 140) (end 99.025 143.525) (width 1) (layer "F.Cu") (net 10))
 (segment (start 99.7877 131.03) (end 98.585619 131.03) (width 1) (layer "F.Cu") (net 10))
 (segment (start 95.5 134.115619) (end 95.5 140) (width 1) (layer "F.Cu") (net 10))
 (segment (start 98.585619 131.03) (end 95.5 134.115619) (width 1) (layer "F.Cu") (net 10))
 (segment (start 115.675 134.975) (end 115.675 117.99) (width 1) (layer "F.Cu") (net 10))
 (segment (start 107.125 143.525) (end 115.675 134.975) (width 1) (layer "F.Cu") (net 10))
 (segment (start 134.4 86.5) (end 130.5 86.5) (width 1) (layer "B.Cu") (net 61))
 (segment (start 137.05 101.695) (end 137.05 89.15) (width 1) (layer "B.Cu") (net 61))
 (segment (start 127 79.08) (end 113.62 65.7) (width 1) (layer "B.Cu") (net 61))
 (segment (start 137.05 89.15) (end 134.4 86.5) (width 1) (layer "B.Cu") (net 61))
 (segment (start 130.5 86.5) (end 127 83) (width 1) (layer "B.Cu") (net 61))
 (segment (start 125.745 113) (end 137.05 101.695) (width 1) (layer "B.Cu") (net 61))
 (segment (start 127 83) (end 127 79.08) (width 1) (layer "B.Cu") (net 61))
 (segment (start 111.5 57) (end 113 55.5) (width 1) (layer "F.Cu") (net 15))
 (segment (start 145.62 114.355) (end 144.175 115.8) (width 1) (layer "F.Cu") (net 15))
 (segment (start 147.5 111.17) (end 145.62 113.05) (width 1) (layer "F.Cu") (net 15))
 (segment (start 144.175 115.8) (end 132.125 115.8) (width 1) (layer "F.Cu") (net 15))
 (segment (start 145.62 113.05) (end 145.62 114.355) (width 1) (layer "F.Cu") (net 15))
 (segment (start 111.5 68.66) (end 111.5 57) (width 1) (layer "F.Cu") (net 15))
 (segment (start 113 55.5) (end 115.5 55.5) (width 1) (layer "F.Cu") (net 15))
 (segment (start 115.5 55.5) (end 129 42) (width 1) (layer "F.Cu") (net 15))
 (segment (start 130.825 114.5) (end 130.825 113) (width 1) (layer "F.Cu") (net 15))
 (segment (start 147.5 45) (end 147.5 111.17) (width 1) (layer "F.Cu") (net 15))
 (segment (start 129 42) (end 144.5 42) (width 1) (layer "F.Cu") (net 15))
 (segment (start 144.5 42) (end 147.5 45) (width 1) (layer "F.Cu") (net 15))
 (segment (start 113.62 70.78) (end 111.5 68.66) (width 1) (layer "F.Cu") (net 15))
 (segment (start 132.125 115.8) (end 130.825 114.5) (width 1) (layer "F.Cu") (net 15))
 (segment (start 113.045 114.77) (end 113.045 113) (width 1) (layer "B.Cu") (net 15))
 (segment (start 114 115.725) (end 113.045 114.77) (width 1) (layer "B.Cu") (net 15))
 (segment (start 130.825 114.6) (end 129.7 115.725) (width 1) (layer "B.Cu") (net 15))
 (segment (start 143.02 115.65) (end 145.62 113.05) (width 1) (layer "B.Cu") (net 15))
 (segment (start 131.6 115.65) (end 143.02 115.65) (width 1) (layer "B.Cu") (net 15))
 (segment (start 130.825 114.6) (end 130.825 114.875) (width 1) (layer "B.Cu") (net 15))
 (segment (start 130.825 114.875) (end 131.6 115.65) (width 1) (layer "B.Cu") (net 15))
 (segment (start 130.825 113) (end 130.825 114.6) (width 1) (layer "B.Cu") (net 15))
 (segment (start 129.7 115.725) (end 114 115.725) (width 1) (layer "B.Cu") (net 15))
 (segment (start 97.5 139.5) (end 99.5 141.5) (width 1) (layer "F.Cu") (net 12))
 (segment (start 112.65 118.475) (end 118.125 113) (width 1) (layer "F.Cu") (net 12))
 (segment (start 112.65 134.85) (end 112.65 118.475) (width 1) (layer "F.Cu") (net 12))
 (segment (start 106 141.5) (end 112.65 134.85) (width 1) (layer "F.Cu") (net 12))
 (segment (start 98.43 133.57) (end 97.5 134.5) (width 1) (layer "F.Cu") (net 12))
 (segment (start 99.5 141.5) (end 106 141.5) (width 1) (layer "F.Cu") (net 12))
 (segment (start 99.7877 133.57) (end 98.43 133.57) (width 1) (layer "F.Cu") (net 12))
 (segment (start 97.5 134.5) (end 97.5 139.5) (width 1) (layer "F.Cu") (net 12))
 (segment (start 127 60.62) (end 130.62 57) (width 1) (layer "B.Cu") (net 3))
 (segment (start 130.62 57) (end 135 57) (width 1) (layer "B.Cu") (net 3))
 (segment (start 148.5 105.09) (end 140.54 113.05) (width 1) (layer "B.Cu") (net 3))
 (segment (start 135 57) (end 148.5 70.5) (width 1) (layer "B.Cu") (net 3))
 (segment (start 148.5 70.5) (end 148.5 105.09) (width 1) (layer "B.Cu") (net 3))
 (segment (start 105.85 127.5077) (end 105.85 113.25) (width 1) (layer "B.Cu") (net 11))
 (segment (start 105.85 113.25) (end 121.15 97.95) (width 1) (layer "B.Cu") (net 11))
 (segment (start 121.15 97.95) (end 132.37 97.95) (width 1) (layer "B.Cu") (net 11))
 (segment (start 132.37 97.95) (end 134.62 95.7) (width 1) (layer "B.Cu") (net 11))
 (segment (start 102.3277 131.03) (end 105.85 127.5077) (width 1) (layer "B.Cu") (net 11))
 (segment (start 108.5 93.2) (end 106 95.7) (width 1) (layer "B.Cu") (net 56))
 (segment (start 132.04 93.2) (end 108.5 93.2) (width 1) (layer "B.Cu") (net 56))
 (segment (start 134.62 90.62) (end 132.04 93.2) (width 1) (layer "B.Cu") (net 56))
 (segment (start 127 53) (end 121.24 53) (width 1) (layer "F.Cu") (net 2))
 (segment (start 121.24 53) (end 113.62 60.62) (width 1) (layer "F.Cu") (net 2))
 (segment (start 113.62 95.7) (end 106.875 102.445) (width 1) (layer "F.Cu") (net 14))
 (segment (start 106.875 102.445) (end 106.875 131.5627) (width 1) (layer "F.Cu") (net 14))
 (segment (start 106.875 131.5627) (end 102.3277 136.11) (width 1) (layer "F.Cu") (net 14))
 (segment (start 113 85.5) (end 116.5 85.5) (width 1) (layer "F.Cu") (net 4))
 (segment (start 107.5 80) (end 113 85.5) (width 1) (layer "F.Cu") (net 4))
 (segment (start 102.3277 133.57) (end 105 130.8977) (width 1) (layer "F.Cu") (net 4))
 (segment (start 103.5 105.5) (end 103.5 95) (width 1) (layer "F.Cu") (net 4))
 (segment (start 118.5 74.2) (end 127 65.7) (width 1) (layer "F.Cu") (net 4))
 (segment (start 116.5 85.5) (end 118.5 83.5) (width 1) (layer "F.Cu") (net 4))
 (segment (start 105 107) (end 103.5 105.5) (width 1) (layer "F.Cu") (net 4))
 (segment (start 100 91.5) (end 100 83.5) (width 1) (layer "F.Cu") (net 4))
 (segment (start 118.5 83.5) (end 118.5 74.2) (width 1) (layer "F.Cu") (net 4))
 (segment (start 103.5 80) (end 107.5 80) (width 1) (layer "F.Cu") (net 4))
 (segment (start 105 130.8977) (end 105 107) (width 1) (layer "F.Cu") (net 4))
 (segment (start 103.5 95) (end 100 91.5) (width 1) (layer "F.Cu") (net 4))
 (segment (start 100 83.5) (end 103.5 80) (width 1) (layer "F.Cu") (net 4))
 (segment (start 102.3277 128.49) (end 102.3277 125.95) (width 1) (layer "F.Cu") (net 7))
 (segment (start 102.3277 119.8277) (end 102.3277 125.95) (width 1) (layer "B.Cu") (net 7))
 (segment (start 92.5 110) (end 102.3277 119.8277) (width 1) (layer "B.Cu") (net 7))
 (segment (start 107 50.5) (end 104 50.5) (width 1) (layer "B.Cu") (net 7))
 (segment (start 92.5 62) (end 92.5 110) (width 1) (layer "B.Cu") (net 7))
 (segment (start 120 63.5) (end 107 50.5) (width 1) (layer "B.Cu") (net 7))
 (segment (start 132.42 63.5) (end 134.62 65.7) (width 1) (layer "B.Cu") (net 7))
 (segment (start 104 50.5) (end 92.5 62) (width 1) (layer "B.Cu") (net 7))
 (segment (start 132.42 63.5) (end 120 63.5) (width 1) (layer "B.Cu") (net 7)))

